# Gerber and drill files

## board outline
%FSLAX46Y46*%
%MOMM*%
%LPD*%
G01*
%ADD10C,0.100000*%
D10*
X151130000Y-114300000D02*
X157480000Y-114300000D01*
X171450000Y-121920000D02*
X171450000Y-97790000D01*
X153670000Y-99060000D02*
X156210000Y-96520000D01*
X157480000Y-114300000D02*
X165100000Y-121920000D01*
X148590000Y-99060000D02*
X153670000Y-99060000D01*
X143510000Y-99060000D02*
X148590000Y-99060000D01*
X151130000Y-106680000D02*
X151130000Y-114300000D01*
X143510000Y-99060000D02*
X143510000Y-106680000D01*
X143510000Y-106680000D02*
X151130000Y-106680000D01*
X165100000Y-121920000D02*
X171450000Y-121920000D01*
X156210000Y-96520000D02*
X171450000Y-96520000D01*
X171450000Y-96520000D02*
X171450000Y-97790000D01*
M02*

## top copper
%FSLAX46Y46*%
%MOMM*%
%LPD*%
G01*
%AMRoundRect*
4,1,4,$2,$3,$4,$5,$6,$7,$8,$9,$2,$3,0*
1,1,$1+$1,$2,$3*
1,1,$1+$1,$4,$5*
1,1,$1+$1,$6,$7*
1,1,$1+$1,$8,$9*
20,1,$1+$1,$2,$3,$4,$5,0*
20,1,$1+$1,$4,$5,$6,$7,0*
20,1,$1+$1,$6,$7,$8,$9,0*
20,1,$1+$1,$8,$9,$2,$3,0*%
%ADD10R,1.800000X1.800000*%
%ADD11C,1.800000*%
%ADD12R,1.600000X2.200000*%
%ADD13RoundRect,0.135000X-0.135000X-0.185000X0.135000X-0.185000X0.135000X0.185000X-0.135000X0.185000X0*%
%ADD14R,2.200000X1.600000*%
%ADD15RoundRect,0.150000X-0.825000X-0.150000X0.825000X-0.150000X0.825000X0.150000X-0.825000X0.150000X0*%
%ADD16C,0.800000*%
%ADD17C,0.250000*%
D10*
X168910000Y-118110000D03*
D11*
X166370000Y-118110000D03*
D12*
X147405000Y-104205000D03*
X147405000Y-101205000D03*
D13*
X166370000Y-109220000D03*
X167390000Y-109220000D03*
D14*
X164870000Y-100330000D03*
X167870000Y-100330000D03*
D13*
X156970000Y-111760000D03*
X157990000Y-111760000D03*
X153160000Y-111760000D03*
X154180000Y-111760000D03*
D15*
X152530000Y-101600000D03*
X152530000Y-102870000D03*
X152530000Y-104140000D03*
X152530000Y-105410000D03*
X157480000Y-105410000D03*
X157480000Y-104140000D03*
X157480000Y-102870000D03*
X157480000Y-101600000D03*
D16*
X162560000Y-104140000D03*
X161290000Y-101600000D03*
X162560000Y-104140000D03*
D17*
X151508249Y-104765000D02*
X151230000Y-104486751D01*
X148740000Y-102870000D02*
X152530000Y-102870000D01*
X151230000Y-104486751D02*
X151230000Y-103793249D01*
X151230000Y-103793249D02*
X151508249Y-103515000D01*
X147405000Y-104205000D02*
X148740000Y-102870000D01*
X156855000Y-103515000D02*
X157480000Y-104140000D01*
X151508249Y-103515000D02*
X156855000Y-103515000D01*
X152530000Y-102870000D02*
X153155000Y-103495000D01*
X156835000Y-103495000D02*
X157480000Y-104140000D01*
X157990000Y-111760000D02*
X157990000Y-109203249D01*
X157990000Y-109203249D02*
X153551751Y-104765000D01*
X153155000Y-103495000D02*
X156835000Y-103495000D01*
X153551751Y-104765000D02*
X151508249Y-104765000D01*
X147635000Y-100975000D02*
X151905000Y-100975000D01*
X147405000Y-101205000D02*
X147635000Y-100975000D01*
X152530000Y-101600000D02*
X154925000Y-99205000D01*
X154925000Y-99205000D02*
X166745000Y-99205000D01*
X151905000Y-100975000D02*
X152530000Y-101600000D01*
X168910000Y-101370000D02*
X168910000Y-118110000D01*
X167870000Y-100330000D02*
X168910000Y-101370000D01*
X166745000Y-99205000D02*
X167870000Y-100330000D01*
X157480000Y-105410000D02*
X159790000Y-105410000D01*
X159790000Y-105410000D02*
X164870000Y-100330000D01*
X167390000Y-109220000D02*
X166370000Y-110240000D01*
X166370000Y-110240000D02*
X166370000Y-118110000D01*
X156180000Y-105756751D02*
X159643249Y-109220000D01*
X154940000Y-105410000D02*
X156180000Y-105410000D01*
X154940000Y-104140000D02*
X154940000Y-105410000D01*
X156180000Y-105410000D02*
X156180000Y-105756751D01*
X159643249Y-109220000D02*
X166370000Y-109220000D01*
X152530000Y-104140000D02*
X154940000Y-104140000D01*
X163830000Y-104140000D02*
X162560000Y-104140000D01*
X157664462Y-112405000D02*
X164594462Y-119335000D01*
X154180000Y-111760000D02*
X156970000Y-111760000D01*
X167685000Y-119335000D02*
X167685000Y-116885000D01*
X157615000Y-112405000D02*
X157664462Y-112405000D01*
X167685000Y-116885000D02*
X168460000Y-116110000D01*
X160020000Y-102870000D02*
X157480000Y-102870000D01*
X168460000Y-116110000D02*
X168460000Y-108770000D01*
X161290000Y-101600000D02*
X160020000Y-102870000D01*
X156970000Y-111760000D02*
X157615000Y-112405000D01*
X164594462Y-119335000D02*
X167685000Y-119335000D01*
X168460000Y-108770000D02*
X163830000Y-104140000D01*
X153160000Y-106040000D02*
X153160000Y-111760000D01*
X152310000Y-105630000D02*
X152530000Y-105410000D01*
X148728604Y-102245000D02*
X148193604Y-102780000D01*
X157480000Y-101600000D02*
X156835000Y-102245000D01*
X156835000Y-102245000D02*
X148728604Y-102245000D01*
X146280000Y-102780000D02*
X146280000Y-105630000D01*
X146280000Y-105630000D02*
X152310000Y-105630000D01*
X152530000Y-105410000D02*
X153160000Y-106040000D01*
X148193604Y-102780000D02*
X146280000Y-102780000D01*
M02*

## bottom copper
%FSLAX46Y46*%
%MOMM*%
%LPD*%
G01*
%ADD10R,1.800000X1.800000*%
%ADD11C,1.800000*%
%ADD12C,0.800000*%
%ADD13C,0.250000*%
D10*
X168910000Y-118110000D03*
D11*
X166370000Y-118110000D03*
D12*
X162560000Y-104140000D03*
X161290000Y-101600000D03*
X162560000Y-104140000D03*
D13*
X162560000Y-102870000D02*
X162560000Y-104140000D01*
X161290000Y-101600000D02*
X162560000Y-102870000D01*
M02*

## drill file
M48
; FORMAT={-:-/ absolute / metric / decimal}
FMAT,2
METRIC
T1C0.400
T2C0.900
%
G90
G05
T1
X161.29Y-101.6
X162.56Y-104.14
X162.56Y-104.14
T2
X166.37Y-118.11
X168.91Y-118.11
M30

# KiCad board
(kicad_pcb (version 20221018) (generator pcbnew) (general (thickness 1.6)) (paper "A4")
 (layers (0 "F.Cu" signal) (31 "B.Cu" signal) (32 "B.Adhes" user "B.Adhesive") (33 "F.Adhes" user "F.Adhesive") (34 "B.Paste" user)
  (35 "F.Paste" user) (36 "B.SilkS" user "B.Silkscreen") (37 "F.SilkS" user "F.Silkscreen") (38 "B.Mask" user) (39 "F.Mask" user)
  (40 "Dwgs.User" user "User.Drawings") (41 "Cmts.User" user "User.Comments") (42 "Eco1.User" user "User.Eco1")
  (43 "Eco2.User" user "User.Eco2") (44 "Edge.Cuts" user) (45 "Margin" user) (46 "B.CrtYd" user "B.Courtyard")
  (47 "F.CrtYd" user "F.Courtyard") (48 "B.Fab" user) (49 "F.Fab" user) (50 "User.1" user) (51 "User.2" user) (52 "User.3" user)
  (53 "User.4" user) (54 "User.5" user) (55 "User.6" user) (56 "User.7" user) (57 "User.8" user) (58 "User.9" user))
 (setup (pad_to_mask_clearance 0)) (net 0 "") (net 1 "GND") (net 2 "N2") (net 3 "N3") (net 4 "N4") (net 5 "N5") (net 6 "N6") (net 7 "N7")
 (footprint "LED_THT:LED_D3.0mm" (layer "F.Cu") (at 168.91 118.11 180)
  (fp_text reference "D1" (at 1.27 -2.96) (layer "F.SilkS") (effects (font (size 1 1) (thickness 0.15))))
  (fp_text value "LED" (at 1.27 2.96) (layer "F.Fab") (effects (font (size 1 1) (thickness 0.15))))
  (pad "1" thru_hole rect (at 0 0 180) (size 1.8 1.8) (drill 0.9) (layers "*.Cu" "*.Mask") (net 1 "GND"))
  (pad "2" thru_hole circle (at 2.54 0 180) (size 1.8 1.8) (drill 0.9) (layers "*.Cu" "*.Mask") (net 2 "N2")))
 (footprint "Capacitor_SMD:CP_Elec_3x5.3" (layer "F.Cu") (at 147.405 102.705 90)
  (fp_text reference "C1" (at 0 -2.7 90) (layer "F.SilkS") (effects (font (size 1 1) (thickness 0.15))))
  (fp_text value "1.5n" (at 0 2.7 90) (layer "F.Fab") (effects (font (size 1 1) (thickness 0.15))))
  (pad "1" smd rect (at -1.5 0 90) (size 2.2 1.6) (layers "F.Cu" "F.Paste" "F.Mask") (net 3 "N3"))
  (pad "2" smd rect (at 1.5 0 90) (size 2.2 1.6) (layers "F.Cu" "F.Paste" "F.Mask") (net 1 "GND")))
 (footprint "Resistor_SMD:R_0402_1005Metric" (layer "F.Cu") (at 166.88 109.22)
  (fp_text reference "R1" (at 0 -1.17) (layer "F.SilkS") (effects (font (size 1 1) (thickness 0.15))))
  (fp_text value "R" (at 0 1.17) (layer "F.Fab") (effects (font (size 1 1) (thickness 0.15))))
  (pad "1" smd roundrect (at -0.51 0) (size 0.54 0.64) (layers "F.Cu" "F.Paste" "F.Mask") (roundrect_rratio 0.25) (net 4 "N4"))
  (pad "2" smd roundrect (at 0.51 0) (size 0.54 0.64) (layers "F.Cu" "F.Paste" "F.Mask") (roundrect_rratio 0.25) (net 2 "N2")))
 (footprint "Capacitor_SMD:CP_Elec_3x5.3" (layer "F.Cu") (at 166.37 100.33)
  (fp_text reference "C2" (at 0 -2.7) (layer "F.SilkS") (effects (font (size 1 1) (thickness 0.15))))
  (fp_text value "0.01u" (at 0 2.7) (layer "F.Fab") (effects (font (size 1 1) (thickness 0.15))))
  (pad "1" smd rect (at -1.5 0) (size 2.2 1.6) (layers "F.Cu" "F.Paste" "F.Mask") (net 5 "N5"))
  (pad "2" smd rect (at 1.5 0) (size 2.2 1.6) (layers "F.Cu" "F.Paste" "F.Mask") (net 1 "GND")))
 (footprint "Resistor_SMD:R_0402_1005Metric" (layer "F.Cu") (at 157.48 111.76)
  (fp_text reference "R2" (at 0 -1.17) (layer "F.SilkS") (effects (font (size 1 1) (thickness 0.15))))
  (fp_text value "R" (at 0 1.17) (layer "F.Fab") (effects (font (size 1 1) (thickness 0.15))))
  (pad "1" smd roundrect (at -0.51 0) (size 0.54 0.64) (layers "F.Cu" "F.Paste" "F.Mask") (roundrect_rratio 0.25) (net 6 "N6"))
  (pad "2" smd roundrect (at 0.51 0) (size 0.54 0.64) (layers "F.Cu" "F.Paste" "F.Mask") (roundrect_rratio 0.25) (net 3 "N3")))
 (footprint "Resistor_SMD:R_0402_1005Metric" (layer "F.Cu") (at 153.67 111.76)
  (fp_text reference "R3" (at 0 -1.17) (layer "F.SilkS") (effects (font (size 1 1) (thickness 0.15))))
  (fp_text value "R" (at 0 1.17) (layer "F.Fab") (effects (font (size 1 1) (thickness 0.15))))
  (pad "1" smd roundrect (at -0.51 0) (size 0.54 0.64) (layers "F.Cu" "F.Paste" "F.Mask") (roundrect_rratio 0.25) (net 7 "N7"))
  (pad "2" smd roundrect (at 0.51 0) (size 0.54 0.64) (layers "F.Cu" "F.Paste" "F.Mask") (roundrect_rratio 0.25) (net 6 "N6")))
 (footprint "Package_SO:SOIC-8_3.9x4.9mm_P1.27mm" (layer "F.Cu") (at 155.005 103.505)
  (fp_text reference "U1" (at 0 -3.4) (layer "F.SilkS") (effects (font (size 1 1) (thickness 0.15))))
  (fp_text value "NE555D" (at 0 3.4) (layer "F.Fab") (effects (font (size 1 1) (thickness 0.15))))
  (pad "1" smd roundrect (at -2.475 -1.905) (size 1.95 0.6) (layers "F.Cu" "F.Paste" "F.Mask") (roundrect_rratio 0.25) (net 1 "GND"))
  (pad "2" smd roundrect (at -2.475 -0.635) (size 1.95 0.6) (layers "F.Cu" "F.Paste" "F.Mask") (roundrect_rratio 0.25) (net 3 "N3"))
  (pad "3" smd roundrect (at -2.475 0.635) (size 1.95 0.6) (layers "F.Cu" "F.Paste" "F.Mask") (roundrect_rratio 0.25) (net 4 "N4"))
  (pad "4" smd roundrect (at -2.475 1.905) (size 1.95 0.6) (layers "F.Cu" "F.Paste" "F.Mask") (roundrect_rratio 0.25) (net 7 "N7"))
  (pad "5" smd roundrect (at 2.475 1.905) (size 1.95 0.6) (layers "F.Cu" "F.Paste" "F.Mask") (roundrect_rratio 0.25) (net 5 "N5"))
  (pad "6" smd roundrect (at 2.475 0.635) (size 1.95 0.6) (layers "F.Cu" "F.Paste" "F.Mask") (roundrect_rratio 0.25) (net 3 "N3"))
  (pad "7" smd roundrect (at 2.475 -0.635) (size 1.95 0.6) (layers "F.Cu" "F.Paste" "F.Mask") (roundrect_rratio 0.25) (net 6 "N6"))
  (pad "8" smd roundrect (at 2.475 -1.905) (size 1.95 0.6) (layers "F.Cu" "F.Paste" "F.Mask") (roundrect_rratio 0.25) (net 7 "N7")))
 (gr_line (start 151.13 114.3) (end 157.48 114.3) (stroke (width 0.1) (type default)) (layer "Edge.Cuts"))
 (gr_line (start 171.45 121.92) (end 171.45 97.79) (stroke (width 0.1) (type default)) (layer "Edge.Cuts"))
 (gr_line (start 153.67 99.06) (end 156.21 96.52) (stroke (width 0.1) (type default)) (layer "Edge.Cuts"))
 (gr_line (start 157.48 114.3) (end 165.1 121.92) (stroke (width 0.1) (type default)) (layer "Edge.Cuts"))
 (gr_line (start 148.59 99.06) (end 153.67 99.06) (stroke (width 0.1) (type default)) (layer "Edge.Cuts"))
 (gr_line (start 143.51 99.06) (end 148.59 99.06) (stroke (width 0.1) (type default)) (layer "Edge.Cuts"))
 (gr_line (start 151.13 106.68) (end 151.13 114.3) (stroke (width 0.1) (type default)) (layer "Edge.Cuts"))
 (gr_line (start 143.51 99.06) (end 143.51 106.68) (stroke (width 0.1) (type default)) (layer "Edge.Cuts"))
 (gr_line (start 143.51 106.68) (end 151.13 106.68) (stroke (width 0.1) (type default)) (layer "Edge.Cuts"))
 (gr_line (start 165.1 121.92) (end 171.45 121.92) (stroke (width 0.1) (type default)) (layer "Edge.Cuts"))
 (gr_line (start 156.21 96.52) (end 171.45 96.52) (stroke (width 0.1) (type default)) (layer "Edge.Cuts"))
 (gr_line (start 171.45 96.52) (end 171.45 97.79) (stroke (width 0.1) (type default)) (layer "Edge.Cuts"))
 (segment (start 151.508249 104.765) (end 151.23 104.486751) (width 0.25) (layer "F.Cu") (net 3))
 (segment (start 148.74 102.87) (end 152.53 102.87) (width 0.25) (layer "F.Cu") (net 3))
 (segment (start 151.23 104.486751) (end 151.23 103.793249) (width 0.25) (layer "F.Cu") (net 3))
 (segment (start 151.23 103.793249) (end 151.508249 103.515) (width 0.25) (layer "F.Cu") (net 3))
 (segment (start 147.405 104.205) (end 148.74 102.87) (width 0.25) (layer "F.Cu") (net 3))
 (segment (start 156.855 103.515) (end 157.48 104.14) (width 0.25) (layer "F.Cu") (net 3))
 (segment (start 151.508249 103.515) (end 156.855 103.515) (width 0.25) (layer "F.Cu") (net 3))
 (segment (start 152.53 102.87) (end 153.155 103.495) (width 0.25) (layer "F.Cu") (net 3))
 (segment (start 156.835 103.495) (end 157.48 104.14) (width 0.25) (layer "F.Cu") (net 3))
 (segment (start 157.99 111.76) (end 157.99 109.203249) (width 0.25) (layer "F.Cu") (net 3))
 (segment (start 157.99 109.203249) (end 153.551751 104.765) (width 0.25) (layer "F.Cu") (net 3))
 (segment (start 153.155 103.495) (end 156.835 103.495) (width 0.25) (layer "F.Cu") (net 3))
 (segment (start 153.551751 104.765) (end 151.508249 104.765) (width 0.25) (layer "F.Cu") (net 3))
 (segment (start 147.635 100.975) (end 151.905 100.975) (width 0.25) (layer "F.Cu") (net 1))
 (segment (start 147.405 101.205) (end 147.635 100.975) (width 0.25) (layer "F.Cu") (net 1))
 (segment (start 152.53 101.6) (end 154.925 99.205) (width 0.25) (layer "F.Cu") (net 1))
 (segment (start 154.925 99.205) (end 166.745 99.205) (width 0.25) (layer "F.Cu") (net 1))
 (segment (start 151.905 100.975) (end 152.53 101.6) (width 0.25) (layer "F.Cu") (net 1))
 (segment (start 168.91 101.37) (end 168.91 118.11) (width 0.25) (layer "F.Cu") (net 1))
 (segment (start 167.87 100.33) (end 168.91 101.37) (width 0.25) (layer "F.Cu") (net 1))
 (segment (start 166.745 99.205) (end 167.87 100.33) (width 0.25) (layer "F.Cu") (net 1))
 (segment (start 157.48 105.41) (end 159.79 105.41) (width 0.25) (layer "F.Cu") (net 5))
 (segment (start 159.79 105.41) (end 164.87 100.33) (width 0.25) (layer "F.Cu") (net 5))
 (segment (start 167.39 109.22) (end 166.37 110.24) (width 0.25) (layer "F.Cu") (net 2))
 (segment (start 166.37 110.24) (end 166.37 118.11) (width 0.25) (layer "F.Cu") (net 2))
 (segment (start 156.18 105.756751) (end 159.643249 109.22) (width 0.25) (layer "F.Cu") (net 4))
 (segment (start 154.94 105.41) (end 156.18 105.41) (width 0.25) (layer "F.Cu") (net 4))
 (segment (start 154.94 104.14) (end 154.94 105.41) (width 0.25) (layer "F.Cu") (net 4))
 (segment (start 156.18 105.41) (end 156.18 105.756751) (width 0.25) (layer "F.Cu") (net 4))
 (segment (start 159.643249 109.22) (end 166.37 109.22) (width 0.25) (layer "F.Cu") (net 4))
 (segment (start 152.53 104.14) (end 154.94 104.14) (width 0.25) (layer "F.Cu") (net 4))
 (segment (start 163.83 104.14) (end 162.56 104.14) (width 0.25) (layer "F.Cu") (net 6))
 (segment (start 157.664462 112.405) (end 164.594462 119.335) (width 0.25) (layer "F.Cu") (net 6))
 (segment (start 154.18 111.76) (end 156.97 111.76) (width 0.25) (layer "F.Cu") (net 6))
 (segment (start 167.685 119.335) (end 167.685 116.885) (width 0.25) (layer "F.Cu") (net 6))
 (segment (start 157.615 112.405) (end 157.664462 112.405) (width 0.25) (layer "F.Cu") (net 6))
 (segment (start 167.685 116.885) (end 168.46 116.11) (width 0.25) (layer "F.Cu") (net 6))
 (segment (start 160.02 102.87) (end 157.48 102.87) (width 0.25) (layer "F.Cu") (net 6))
 (segment (start 168.46 116.11) (end 168.46 108.77) (width 0.25) (layer "F.Cu") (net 6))
 (segment (start 161.29 101.6) (end 160.02 102.87) (width 0.25) (layer "F.Cu") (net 6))
 (segment (start 156.97 111.76) (end 157.615 112.405) (width 0.25) (layer "F.Cu") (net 6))
 (segment (start 164.594462 119.335) (end 167.685 119.335) (width 0.25) (layer "F.Cu") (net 6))
 (segment (start 168.46 108.77) (end 163.83 104.14) (width 0.25) (layer "F.Cu") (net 6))
 (via (at 162.56 104.14) (size 0.8) (drill 0.4) (layers "F.Cu" "B.Cu") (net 6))
 (via (at 161.29 101.6) (size 0.8) (drill 0.4) (layers "F.Cu" "B.Cu") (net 6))
 (via (at 162.56 104.14) (size 0.8) (drill 0.4) (layers "F.Cu" "B.Cu") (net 6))
 (segment (start 162.56 102.87) (end 162.56 104.14) (width 0.25) (layer "B.Cu") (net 6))
 (segment (start 161.29 101.6) (end 162.56 102.87) (width 0.25) (layer "B.Cu") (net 6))
 (segment (start 153.16 106.04) (end 153.16 111.76) (width 0.25) (layer "F.Cu") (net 7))
 (segment (start 152.31 105.63) (end 152.53 105.41) (width 0.25) (layer "F.Cu") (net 7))
 (segment (start 148.728604 102.245) (end 148.193604 102.78) (width 0.25) (layer "F.Cu") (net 7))
 (segment (start 157.48 101.6) (end 156.835 102.245) (width 0.25) (layer "F.Cu") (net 7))
 (segment (start 156.835 102.245) (end 148.728604 102.245) (width 0.25) (layer "F.Cu") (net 7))
 (segment (start 146.28 102.78) (end 146.28 105.63) (width 0.25) (layer "F.Cu") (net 7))
 (segment (start 146.28 105.63) (end 152.31 105.63) (width 0.25) (layer "F.Cu") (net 7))
 (segment (start 152.53 105.41) (end 153.16 106.04) (width 0.25) (layer "F.Cu") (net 7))
 (segment (start 148.193604 102.78) (end 146.28 102.78) (width 0.25) (layer "F.Cu") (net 7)))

